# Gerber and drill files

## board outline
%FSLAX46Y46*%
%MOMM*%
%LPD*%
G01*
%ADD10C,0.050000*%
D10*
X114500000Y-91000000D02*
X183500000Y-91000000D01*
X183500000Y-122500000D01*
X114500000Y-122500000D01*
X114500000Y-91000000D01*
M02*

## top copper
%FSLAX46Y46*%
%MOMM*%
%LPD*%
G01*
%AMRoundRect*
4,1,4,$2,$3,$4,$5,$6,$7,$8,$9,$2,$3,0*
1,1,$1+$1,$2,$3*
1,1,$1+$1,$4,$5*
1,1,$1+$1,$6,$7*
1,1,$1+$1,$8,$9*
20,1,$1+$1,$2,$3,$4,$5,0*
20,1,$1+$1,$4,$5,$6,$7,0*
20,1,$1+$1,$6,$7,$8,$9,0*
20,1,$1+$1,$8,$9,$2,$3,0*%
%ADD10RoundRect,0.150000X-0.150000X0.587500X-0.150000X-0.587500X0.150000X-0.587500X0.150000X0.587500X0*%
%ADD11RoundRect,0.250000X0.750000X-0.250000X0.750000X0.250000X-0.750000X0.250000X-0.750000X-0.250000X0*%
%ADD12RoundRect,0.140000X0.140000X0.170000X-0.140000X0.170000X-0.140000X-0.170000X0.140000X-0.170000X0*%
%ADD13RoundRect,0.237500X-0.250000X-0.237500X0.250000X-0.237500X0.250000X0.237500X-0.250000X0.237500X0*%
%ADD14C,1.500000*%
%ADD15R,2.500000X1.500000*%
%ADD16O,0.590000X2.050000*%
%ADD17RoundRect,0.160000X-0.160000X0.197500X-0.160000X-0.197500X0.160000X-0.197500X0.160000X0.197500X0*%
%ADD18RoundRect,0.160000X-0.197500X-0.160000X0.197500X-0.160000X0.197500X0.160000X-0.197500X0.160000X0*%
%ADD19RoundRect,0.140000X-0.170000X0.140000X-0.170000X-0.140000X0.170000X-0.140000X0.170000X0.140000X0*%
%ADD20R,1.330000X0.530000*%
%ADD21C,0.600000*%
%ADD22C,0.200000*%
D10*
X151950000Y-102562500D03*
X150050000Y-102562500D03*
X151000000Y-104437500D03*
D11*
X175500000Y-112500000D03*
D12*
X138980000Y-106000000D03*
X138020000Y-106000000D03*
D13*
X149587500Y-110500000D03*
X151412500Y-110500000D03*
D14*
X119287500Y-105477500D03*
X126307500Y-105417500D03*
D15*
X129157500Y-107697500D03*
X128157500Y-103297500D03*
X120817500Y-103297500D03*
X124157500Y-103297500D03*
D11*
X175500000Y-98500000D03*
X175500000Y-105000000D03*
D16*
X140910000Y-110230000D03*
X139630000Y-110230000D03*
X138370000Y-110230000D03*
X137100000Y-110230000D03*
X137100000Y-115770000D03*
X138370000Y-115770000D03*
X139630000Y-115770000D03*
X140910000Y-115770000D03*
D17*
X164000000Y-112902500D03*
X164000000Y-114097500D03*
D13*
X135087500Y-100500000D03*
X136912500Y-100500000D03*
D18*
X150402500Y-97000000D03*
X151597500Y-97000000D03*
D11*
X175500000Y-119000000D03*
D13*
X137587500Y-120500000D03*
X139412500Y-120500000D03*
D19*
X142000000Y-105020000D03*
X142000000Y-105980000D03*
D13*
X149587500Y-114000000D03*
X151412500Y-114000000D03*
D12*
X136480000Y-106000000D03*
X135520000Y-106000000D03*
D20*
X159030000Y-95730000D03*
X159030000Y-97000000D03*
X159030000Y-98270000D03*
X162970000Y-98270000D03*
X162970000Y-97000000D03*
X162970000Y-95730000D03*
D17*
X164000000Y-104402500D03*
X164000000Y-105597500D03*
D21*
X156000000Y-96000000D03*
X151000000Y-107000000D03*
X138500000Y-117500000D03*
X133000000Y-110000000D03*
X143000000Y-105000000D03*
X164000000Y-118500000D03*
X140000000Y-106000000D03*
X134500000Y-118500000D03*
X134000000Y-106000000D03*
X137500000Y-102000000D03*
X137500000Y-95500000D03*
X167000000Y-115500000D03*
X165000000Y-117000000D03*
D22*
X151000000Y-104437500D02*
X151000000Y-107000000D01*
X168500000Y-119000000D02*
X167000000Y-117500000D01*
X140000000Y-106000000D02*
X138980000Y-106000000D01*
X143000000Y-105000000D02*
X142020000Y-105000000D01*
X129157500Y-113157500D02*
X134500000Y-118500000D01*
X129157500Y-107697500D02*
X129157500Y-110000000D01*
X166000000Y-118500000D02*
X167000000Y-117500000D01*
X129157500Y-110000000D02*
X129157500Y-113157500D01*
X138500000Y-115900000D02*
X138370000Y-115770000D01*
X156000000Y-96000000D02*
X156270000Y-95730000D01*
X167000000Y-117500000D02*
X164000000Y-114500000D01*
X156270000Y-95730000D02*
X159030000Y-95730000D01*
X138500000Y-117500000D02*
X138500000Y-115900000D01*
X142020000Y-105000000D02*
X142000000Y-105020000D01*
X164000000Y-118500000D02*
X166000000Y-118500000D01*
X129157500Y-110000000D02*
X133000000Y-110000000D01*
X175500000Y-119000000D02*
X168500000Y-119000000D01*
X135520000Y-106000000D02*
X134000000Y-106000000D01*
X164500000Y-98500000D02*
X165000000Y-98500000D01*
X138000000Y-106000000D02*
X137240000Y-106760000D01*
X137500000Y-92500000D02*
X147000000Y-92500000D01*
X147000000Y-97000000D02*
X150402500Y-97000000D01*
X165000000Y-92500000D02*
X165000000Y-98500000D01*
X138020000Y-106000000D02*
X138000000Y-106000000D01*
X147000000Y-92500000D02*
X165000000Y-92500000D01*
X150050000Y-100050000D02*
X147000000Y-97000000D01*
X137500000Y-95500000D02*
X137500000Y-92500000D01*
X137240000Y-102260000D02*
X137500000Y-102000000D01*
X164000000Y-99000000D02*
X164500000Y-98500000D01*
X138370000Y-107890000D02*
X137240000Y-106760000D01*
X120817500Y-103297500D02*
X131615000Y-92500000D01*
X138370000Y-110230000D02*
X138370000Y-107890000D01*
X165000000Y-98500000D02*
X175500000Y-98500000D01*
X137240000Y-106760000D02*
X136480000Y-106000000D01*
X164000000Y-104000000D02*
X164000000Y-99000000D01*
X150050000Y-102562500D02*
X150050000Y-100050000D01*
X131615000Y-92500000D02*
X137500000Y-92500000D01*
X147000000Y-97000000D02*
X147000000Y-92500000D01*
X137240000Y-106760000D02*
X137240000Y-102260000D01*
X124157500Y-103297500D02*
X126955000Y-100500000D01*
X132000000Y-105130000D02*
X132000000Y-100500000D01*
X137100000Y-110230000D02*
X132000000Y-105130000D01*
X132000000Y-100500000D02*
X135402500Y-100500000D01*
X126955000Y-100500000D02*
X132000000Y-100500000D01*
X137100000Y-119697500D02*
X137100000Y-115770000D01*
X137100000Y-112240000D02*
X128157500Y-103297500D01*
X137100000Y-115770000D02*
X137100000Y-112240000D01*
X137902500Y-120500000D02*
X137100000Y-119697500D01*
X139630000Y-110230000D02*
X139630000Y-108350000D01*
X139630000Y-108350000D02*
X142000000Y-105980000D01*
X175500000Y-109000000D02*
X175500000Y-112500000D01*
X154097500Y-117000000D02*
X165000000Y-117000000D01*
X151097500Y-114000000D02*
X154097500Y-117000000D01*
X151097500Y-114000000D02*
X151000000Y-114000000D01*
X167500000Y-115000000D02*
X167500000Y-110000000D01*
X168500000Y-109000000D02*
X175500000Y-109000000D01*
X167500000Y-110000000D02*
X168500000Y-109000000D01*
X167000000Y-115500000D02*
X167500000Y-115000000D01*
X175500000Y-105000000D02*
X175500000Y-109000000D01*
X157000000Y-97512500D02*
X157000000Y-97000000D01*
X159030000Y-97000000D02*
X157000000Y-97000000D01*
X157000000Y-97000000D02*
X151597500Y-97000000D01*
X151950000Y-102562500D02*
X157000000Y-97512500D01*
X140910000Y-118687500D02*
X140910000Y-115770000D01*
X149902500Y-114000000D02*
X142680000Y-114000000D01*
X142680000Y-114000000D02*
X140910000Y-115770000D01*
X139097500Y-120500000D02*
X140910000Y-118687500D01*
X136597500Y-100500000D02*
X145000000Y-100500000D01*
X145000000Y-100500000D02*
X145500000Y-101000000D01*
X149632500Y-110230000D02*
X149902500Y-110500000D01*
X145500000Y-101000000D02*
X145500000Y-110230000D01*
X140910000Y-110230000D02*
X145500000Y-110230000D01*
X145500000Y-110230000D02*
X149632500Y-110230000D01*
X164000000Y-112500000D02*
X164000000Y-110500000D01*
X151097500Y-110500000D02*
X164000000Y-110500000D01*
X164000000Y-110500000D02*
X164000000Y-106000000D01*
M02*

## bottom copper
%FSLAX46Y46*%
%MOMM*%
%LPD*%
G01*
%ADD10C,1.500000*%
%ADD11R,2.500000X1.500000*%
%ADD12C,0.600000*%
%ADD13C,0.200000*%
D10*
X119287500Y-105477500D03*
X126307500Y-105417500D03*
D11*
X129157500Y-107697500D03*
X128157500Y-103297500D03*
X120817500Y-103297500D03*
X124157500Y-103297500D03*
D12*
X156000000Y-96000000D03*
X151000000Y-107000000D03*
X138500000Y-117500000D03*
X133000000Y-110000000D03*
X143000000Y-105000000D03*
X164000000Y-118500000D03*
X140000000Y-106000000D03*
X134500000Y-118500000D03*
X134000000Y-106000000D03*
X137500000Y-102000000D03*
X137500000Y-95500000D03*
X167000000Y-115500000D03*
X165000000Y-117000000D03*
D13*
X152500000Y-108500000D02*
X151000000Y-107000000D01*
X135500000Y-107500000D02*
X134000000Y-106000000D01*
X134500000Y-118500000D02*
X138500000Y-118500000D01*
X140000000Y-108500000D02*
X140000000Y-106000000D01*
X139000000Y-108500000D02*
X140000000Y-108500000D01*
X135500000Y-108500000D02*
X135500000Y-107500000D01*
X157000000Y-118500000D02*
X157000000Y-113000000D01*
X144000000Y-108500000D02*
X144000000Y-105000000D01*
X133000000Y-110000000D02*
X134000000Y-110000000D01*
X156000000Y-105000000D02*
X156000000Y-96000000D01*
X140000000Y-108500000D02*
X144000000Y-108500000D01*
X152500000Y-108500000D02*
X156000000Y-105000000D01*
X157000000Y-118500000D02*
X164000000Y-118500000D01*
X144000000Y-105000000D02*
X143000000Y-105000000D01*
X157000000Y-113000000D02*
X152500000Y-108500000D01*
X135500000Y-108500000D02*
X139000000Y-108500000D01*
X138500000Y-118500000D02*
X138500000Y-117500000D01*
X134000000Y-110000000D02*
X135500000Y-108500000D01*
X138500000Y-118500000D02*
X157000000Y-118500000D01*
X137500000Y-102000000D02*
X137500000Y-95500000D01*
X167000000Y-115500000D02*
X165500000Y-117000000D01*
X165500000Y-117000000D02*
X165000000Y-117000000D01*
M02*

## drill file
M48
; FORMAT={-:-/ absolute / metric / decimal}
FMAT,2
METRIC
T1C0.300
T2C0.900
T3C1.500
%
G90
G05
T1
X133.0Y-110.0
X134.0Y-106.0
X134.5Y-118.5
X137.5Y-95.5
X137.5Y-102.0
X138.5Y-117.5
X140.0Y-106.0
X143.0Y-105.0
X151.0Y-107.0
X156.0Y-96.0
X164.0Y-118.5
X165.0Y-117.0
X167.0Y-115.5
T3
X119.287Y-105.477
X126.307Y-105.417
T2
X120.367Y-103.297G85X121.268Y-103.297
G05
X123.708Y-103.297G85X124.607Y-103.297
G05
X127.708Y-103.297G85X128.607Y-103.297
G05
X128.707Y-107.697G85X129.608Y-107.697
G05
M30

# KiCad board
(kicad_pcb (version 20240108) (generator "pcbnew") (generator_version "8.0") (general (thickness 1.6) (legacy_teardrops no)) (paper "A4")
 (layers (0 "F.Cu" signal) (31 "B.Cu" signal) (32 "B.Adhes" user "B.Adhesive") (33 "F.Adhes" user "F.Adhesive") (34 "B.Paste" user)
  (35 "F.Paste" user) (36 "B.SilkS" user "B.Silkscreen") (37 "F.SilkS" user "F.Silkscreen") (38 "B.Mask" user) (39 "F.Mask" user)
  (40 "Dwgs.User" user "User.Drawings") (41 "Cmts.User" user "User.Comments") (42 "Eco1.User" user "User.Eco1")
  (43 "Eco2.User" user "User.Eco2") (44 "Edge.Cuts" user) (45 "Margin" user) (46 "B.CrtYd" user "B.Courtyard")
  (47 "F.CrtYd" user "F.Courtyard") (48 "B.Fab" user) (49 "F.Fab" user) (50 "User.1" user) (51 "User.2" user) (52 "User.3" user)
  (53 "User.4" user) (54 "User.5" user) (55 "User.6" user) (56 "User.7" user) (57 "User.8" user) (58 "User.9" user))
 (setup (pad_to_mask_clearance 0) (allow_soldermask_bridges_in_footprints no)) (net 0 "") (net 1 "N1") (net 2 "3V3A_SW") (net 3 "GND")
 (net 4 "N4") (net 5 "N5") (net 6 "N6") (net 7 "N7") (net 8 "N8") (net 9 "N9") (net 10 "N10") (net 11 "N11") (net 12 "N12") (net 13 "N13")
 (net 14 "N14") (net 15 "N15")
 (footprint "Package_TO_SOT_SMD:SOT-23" (layer "F.Cu") (at 151 103.5 -90)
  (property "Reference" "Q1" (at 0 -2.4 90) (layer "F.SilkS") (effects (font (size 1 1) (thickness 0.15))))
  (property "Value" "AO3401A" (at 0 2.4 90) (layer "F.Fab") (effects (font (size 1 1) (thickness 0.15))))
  (pad "1" smd roundrect (at -0.9375 -0.95 270) (size 1.475 0.6) (layers "F.Cu" "F.Paste" "F.Mask") (roundrect_rratio 0.25) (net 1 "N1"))
  (pad "2" smd roundrect (at -0.9375 0.95 270) (size 1.475 0.6) (layers "F.Cu" "F.Paste" "F.Mask") (roundrect_rratio 0.25) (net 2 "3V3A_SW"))
  (pad "3" smd roundrect (at 0.9375 0 270) (size 1.475 0.6) (layers "F.Cu" "F.Paste" "F.Mask") (roundrect_rratio 0.25) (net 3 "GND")))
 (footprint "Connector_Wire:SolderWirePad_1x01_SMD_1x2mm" (layer "F.Cu") (at 175.5 112.5 90)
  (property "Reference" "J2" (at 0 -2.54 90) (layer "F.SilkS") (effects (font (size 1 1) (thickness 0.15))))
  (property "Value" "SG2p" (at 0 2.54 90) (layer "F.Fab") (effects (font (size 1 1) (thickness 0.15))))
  (pad "1" smd roundrect (at 0 0 90) (size 1 2) (layers "F.Cu" "F.Paste" "F.Mask") (roundrect_rratio 0.25) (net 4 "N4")))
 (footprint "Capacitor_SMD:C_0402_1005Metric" (layer "F.Cu") (at 138.5 106 180)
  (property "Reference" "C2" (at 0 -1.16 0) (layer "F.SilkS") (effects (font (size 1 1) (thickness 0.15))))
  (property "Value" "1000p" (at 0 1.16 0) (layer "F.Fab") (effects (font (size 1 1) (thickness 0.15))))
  (pad "1" smd roundrect (at -0.48 0 180) (size 0.56 0.62) (layers "F.Cu" "F.Paste" "F.Mask") (roundrect_rratio 0.25) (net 3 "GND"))
  (pad "2" smd roundrect (at 0.48 0 180) (size 0.56 0.62) (layers "F.Cu" "F.Paste" "F.Mask") (roundrect_rratio 0.25) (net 2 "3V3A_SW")))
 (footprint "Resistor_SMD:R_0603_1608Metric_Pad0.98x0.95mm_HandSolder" (layer "F.Cu") (at 150.5 110.5)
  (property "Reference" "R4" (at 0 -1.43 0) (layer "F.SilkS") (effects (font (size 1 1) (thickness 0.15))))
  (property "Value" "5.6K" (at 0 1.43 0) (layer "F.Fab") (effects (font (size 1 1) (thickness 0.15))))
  (pad "1" smd roundrect (at -0.9125 0) (size 0.975 0.95) (layers "F.Cu" "F.Paste" "F.Mask") (roundrect_rratio 0.25) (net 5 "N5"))
  (pad "2" smd roundrect (at 0.9125 0) (size 0.975 0.95) (layers "F.Cu" "F.Paste" "F.Mask") (roundrect_rratio 0.25) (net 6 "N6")))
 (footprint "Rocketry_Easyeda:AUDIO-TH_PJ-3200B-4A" (layer "F.Cu") (at 124.9875 105.4975)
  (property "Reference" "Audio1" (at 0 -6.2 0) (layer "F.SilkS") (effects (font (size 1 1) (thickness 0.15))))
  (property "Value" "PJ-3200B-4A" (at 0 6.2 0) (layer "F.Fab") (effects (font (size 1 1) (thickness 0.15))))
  (pad "" thru_hole circle (at -5.7 -0.02) (size 1.5 1.5) (drill 1.5) (layers "*.Cu" "*.Mask") (remove_unused_layers no))
  (pad "" thru_hole circle (at 1.32 -0.08) (size 1.5 1.5) (drill 1.5) (layers "*.Cu" "*.Mask") (remove_unused_layers no))
  (pad "1" thru_hole rect (at 4.17 2.2 90) (size 1.5 2.5) (drill oval 0.900024 1.8002) (layers "*.Cu" "*.Mask") (remove_unused_layers no)
   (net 3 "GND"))
  (pad "2" thru_hole rect (at 3.17 -2.2 90) (size 1.5 2.5) (drill oval 0.900024 1.799946) (layers "*.Cu" "*.Mask") (remove_unused_layers no)
   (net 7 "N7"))
  (pad "3" thru_hole rect (at -4.17 -2.2 90) (size 1.5 2.5) (drill oval 0.900024 1.8002) (layers "*.Cu" "*.Mask") (remove_unused_layers no)
   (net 2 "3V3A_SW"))
  (pad "4" thru_hole rect (at -0.83 -2.2 90) (size 1.5 2.5) (drill oval 0.900024 1.799946) (layers "*.Cu" "*.Mask")
   (remove_unused_layers no) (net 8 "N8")))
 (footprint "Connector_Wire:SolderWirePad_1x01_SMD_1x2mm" (layer "F.Cu") (at 175.5 98.5 90)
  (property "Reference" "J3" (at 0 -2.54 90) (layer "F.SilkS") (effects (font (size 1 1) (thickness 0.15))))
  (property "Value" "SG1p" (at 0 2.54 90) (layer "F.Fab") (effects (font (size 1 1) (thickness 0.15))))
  (pad "1" smd roundrect (at 0 0 90) (size 1 2) (layers "F.Cu" "F.Paste" "F.Mask") (roundrect_rratio 0.25) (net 2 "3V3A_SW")))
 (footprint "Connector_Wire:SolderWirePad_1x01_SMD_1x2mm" (layer "F.Cu") (at 175.5 105 90)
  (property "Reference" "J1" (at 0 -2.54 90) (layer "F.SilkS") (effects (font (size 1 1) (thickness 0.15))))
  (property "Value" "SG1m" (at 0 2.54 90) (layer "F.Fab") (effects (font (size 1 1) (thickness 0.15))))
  (pad "1" smd roundrect (at 0 0 90) (size 1 2) (layers "F.Cu" "F.Paste" "F.Mask") (roundrect_rratio 0.25) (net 4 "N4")))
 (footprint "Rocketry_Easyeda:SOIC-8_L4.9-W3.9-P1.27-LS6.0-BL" (layer "F.Cu") (at 139 113 180)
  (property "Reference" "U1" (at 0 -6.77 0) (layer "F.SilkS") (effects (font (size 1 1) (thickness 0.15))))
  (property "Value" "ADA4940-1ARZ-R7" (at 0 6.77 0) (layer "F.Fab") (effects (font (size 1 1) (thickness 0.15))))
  (pad "1" smd oval (at -1.91 2.77 180) (size 0.59 2.05) (layers "F.Cu" "F.Paste" "F.Mask") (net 5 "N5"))
  (pad "2" smd oval (at -0.63 2.77 180) (size 0.59 2.05) (layers "F.Cu" "F.Paste" "F.Mask") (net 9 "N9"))
  (pad "3" smd oval (at 0.63 2.77 180) (size 0.59 2.05) (layers "F.Cu" "F.Paste" "F.Mask") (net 2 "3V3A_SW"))
  (pad "4" smd oval (at 1.9 2.77 180) (size 0.59 2.05) (layers "F.Cu" "F.Paste" "F.Mask") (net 8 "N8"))
  (pad "5" smd oval (at 1.9 -2.77 180) (size 0.59 2.05) (layers "F.Cu" "F.Paste" "F.Mask") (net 7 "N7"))
  (pad "6" smd oval (at 0.63 -2.77 180) (size 0.59 2.05) (layers "F.Cu" "F.Paste" "F.Mask") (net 3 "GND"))
  (pad "7" smd oval (at -0.63 -2.77 180) (size 0.59 2.05) (layers "F.Cu" "F.Paste" "F.Mask") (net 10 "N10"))
  (pad "8" smd oval (at -1.91 -2.77 180) (size 0.59 2.05) (layers "F.Cu" "F.Paste" "F.Mask") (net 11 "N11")))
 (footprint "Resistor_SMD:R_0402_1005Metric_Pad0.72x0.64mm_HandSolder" (layer "F.Cu") (at 164 113.5 -90)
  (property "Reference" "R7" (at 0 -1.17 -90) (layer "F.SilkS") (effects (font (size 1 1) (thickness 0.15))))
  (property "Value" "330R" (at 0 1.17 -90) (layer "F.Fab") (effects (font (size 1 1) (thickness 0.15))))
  (pad "1" smd roundrect (at -0.5975 0 270) (size 0.715 0.64) (layers "F.Cu" "F.Paste" "F.Mask") (roundrect_rratio 0.25) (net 6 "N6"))
  (pad "2" smd roundrect (at 0.5975 0 270) (size 0.715 0.64) (layers "F.Cu" "F.Paste" "F.Mask") (roundrect_rratio 0.25) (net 3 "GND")))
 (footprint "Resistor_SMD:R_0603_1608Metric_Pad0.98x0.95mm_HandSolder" (layer "F.Cu") (at 136 100.5)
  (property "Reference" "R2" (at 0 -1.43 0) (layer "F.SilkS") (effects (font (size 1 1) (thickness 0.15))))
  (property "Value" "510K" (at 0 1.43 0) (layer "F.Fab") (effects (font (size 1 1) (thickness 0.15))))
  (pad "1" smd roundrect (at -0.9125 0) (size 0.975 0.95) (layers "F.Cu" "F.Paste" "F.Mask") (roundrect_rratio 0.25) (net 8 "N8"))
  (pad "2" smd roundrect (at 0.9125 0) (size 0.975 0.95) (layers "F.Cu" "F.Paste" "F.Mask") (roundrect_rratio 0.25) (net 5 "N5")))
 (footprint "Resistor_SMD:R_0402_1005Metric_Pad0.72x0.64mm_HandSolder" (layer "F.Cu") (at 151 97)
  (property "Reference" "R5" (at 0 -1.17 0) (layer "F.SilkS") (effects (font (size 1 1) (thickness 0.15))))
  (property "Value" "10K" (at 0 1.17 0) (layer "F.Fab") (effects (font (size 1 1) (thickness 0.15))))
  (pad "1" smd roundrect (at -0.5975 0) (size 0.715 0.64) (layers "F.Cu" "F.Paste" "F.Mask") (roundrect_rratio 0.25) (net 2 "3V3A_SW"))
  (pad "2" smd roundrect (at 0.5975 0) (size 0.715 0.64) (layers "F.Cu" "F.Paste" "F.Mask") (roundrect_rratio 0.25) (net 1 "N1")))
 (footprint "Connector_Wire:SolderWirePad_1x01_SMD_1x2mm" (layer "F.Cu") (at 175.5 119 90)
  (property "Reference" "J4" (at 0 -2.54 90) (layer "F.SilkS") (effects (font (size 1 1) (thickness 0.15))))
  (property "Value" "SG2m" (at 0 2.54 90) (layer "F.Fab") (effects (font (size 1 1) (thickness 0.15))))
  (pad "1" smd roundrect (at 0 0 90) (size 1 2) (layers "F.Cu" "F.Paste" "F.Mask") (roundrect_rratio 0.25) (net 3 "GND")))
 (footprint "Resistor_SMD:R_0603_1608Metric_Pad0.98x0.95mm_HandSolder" (layer "F.Cu") (at 138.5 120.5)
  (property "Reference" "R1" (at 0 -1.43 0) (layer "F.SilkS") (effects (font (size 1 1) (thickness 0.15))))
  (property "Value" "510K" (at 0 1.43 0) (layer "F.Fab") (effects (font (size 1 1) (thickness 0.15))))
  (pad "1" smd roundrect (at -0.9125 0) (size 0.975 0.95) (layers "F.Cu" "F.Paste" "F.Mask") (roundrect_rratio 0.25) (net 7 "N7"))
  (pad "2" smd roundrect (at 0.9125 0) (size 0.975 0.95) (layers "F.Cu" "F.Paste" "F.Mask") (roundrect_rratio 0.25) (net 11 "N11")))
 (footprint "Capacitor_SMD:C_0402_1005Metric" (layer "F.Cu") (at 142 105.5 -90)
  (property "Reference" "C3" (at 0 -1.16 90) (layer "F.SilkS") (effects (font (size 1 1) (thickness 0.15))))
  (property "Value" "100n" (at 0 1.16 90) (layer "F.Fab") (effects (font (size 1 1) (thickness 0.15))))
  (pad "1" smd roundrect (at -0.48 0 270) (size 0.56 0.62) (layers "F.Cu" "F.Paste" "F.Mask") (roundrect_rratio 0.25) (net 3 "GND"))
  (pad "2" smd roundrect (at 0.48 0 270) (size 0.56 0.62) (layers "F.Cu" "F.Paste" "F.Mask") (roundrect_rratio 0.25) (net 9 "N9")))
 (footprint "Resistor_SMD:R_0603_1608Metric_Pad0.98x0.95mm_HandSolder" (layer "F.Cu") (at 150.5 114)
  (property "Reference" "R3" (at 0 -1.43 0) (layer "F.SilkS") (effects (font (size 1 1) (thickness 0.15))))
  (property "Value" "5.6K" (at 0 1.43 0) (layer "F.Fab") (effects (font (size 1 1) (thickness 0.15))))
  (pad "1" smd roundrect (at -0.9125 0) (size 0.975 0.95) (layers "F.Cu" "F.Paste" "F.Mask") (roundrect_rratio 0.25) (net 11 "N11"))
  (pad "2" smd roundrect (at 0.9125 0) (size 0.975 0.95) (layers "F.Cu" "F.Paste" "F.Mask") (roundrect_rratio 0.25) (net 4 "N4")))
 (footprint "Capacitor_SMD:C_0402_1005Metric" (layer "F.Cu") (at 136 106 180)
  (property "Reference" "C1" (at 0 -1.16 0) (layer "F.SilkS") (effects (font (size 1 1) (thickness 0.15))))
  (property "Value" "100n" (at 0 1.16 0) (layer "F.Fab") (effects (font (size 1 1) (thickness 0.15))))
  (pad "1" smd roundrect (at -0.48 0 180) (size 0.56 0.62) (layers "F.Cu" "F.Paste" "F.Mask") (roundrect_rratio 0.25) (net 2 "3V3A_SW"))
  (pad "2" smd roundrect (at 0.48 0 180) (size 0.56 0.62) (layers "F.Cu" "F.Paste" "F.Mask") (roundrect_rratio 0.25) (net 3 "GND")))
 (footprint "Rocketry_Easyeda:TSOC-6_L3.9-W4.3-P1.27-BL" (layer "F.Cu") (at 161 97 -90)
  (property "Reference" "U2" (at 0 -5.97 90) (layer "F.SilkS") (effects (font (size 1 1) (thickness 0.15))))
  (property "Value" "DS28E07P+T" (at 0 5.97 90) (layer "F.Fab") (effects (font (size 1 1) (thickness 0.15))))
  (pad "1" smd rect (at -1.27 1.97 270) (size 0.53 1.33) (layers "F.Cu" "F.Paste" "F.Mask") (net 3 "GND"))
  (pad "2" smd rect (at 0 1.97 270) (size 0.53 1.33) (layers "F.Cu" "F.Paste" "F.Mask") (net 1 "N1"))
  (pad "3" smd rect (at 1.27 1.97 270) (size 0.53 1.33) (layers "F.Cu" "F.Paste" "F.Mask") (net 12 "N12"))
  (pad "4" smd rect (at 1.27 -1.97 270) (size 0.53 1.33) (layers "F.Cu" "F.Paste" "F.Mask") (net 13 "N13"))
  (pad "5" smd rect (at 0 -1.97 270) (size 0.53 1.33) (layers "F.Cu" "F.Paste" "F.Mask") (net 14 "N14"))
  (pad "6" smd rect (at -1.27 -1.97 270) (size 0.53 1.33) (layers "F.Cu" "F.Paste" "F.Mask") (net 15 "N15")))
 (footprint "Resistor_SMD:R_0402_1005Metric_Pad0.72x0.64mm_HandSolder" (layer "F.Cu") (at 164 105 -90)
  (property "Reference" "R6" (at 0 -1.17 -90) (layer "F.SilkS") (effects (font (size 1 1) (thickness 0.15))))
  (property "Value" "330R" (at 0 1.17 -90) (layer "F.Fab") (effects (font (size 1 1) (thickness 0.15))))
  (pad "1" smd roundrect (at -0.5975 0 270) (size 0.715 0.64) (layers "F.Cu" "F.Paste" "F.Mask") (roundrect_rratio 0.25) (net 2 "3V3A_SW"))
  (pad "2" smd roundrect (at 0.5975 0 270) (size 0.715 0.64) (layers "F.Cu" "F.Paste" "F.Mask") (roundrect_rratio 0.25) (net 6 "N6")))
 (gr_rect (start 114.5 91) (end 183.5 122.5) (stroke (width 0.05) (type default)) (fill none) (layer "Edge.Cuts"))
 (segment (start 151 104.4375) (end 151 107) (width 0.2) (layer "F.Cu") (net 3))
 (segment (start 168.5 119) (end 167 117.5) (width 0.2) (layer "F.Cu") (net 3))
 (segment (start 140 106) (end 138.98 106) (width 0.2) (layer "F.Cu") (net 3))
 (segment (start 143 105) (end 142.02 105) (width 0.2) (layer "F.Cu") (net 3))
 (segment (start 129.1575 113.1575) (end 134.5 118.5) (width 0.2) (layer "F.Cu") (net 3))
 (segment (start 129.1575 107.6975) (end 129.1575 110) (width 0.2) (layer "F.Cu") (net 3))
 (segment (start 166 118.5) (end 167 117.5) (width 0.2) (layer "F.Cu") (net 3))
 (segment (start 129.1575 110) (end 129.1575 113.1575) (width 0.2) (layer "F.Cu") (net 3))
 (segment (start 138.5 115.9) (end 138.37 115.77) (width 0.2) (layer "F.Cu") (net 3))
 (segment (start 156 96) (end 156.27 95.73) (width 0.2) (layer "F.Cu") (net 3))
 (segment (start 167 117.5) (end 164 114.5) (width 0.2) (layer "F.Cu") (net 3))
 (segment (start 156.27 95.73) (end 159.03 95.73) (width 0.2) (layer "F.Cu") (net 3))
 (segment (start 138.5 117.5) (end 138.5 115.9) (width 0.2) (layer "F.Cu") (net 3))
 (segment (start 142.02 105) (end 142 105.02) (width 0.2) (layer "F.Cu") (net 3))
 (segment (start 164 118.5) (end 166 118.5) (width 0.2) (layer "F.Cu") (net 3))
 (segment (start 129.1575 110) (end 133 110) (width 0.2) (layer "F.Cu") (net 3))
 (segment (start 175.5 119) (end 168.5 119) (width 0.2) (layer "F.Cu") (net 3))
 (segment (start 135.52 106) (end 134 106) (width 0.2) (layer "F.Cu") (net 3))
 (via (at 156 96) (size 0.6) (drill 0.3) (layers "F.Cu" "B.Cu") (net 3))
 (via (at 151 107) (size 0.6) (drill 0.3) (layers "F.Cu" "B.Cu") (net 3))
 (via (at 138.5 117.5) (size 0.6) (drill 0.3) (layers "F.Cu" "B.Cu") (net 3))
 (via (at 133 110) (size 0.6) (drill 0.3) (layers "F.Cu" "B.Cu") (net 3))
 (via (at 143 105) (size 0.6) (drill 0.3) (layers "F.Cu" "B.Cu") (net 3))
 (via (at 164 118.5) (size 0.6) (drill 0.3) (layers "F.Cu" "B.Cu") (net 3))
 (via (at 140 106) (size 0.6) (drill 0.3) (layers "F.Cu" "B.Cu") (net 3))
 (via (at 134.5 118.5) (size 0.6) (drill 0.3) (layers "F.Cu" "B.Cu") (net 3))
 (via (at 134 106) (size 0.6) (drill 0.3) (layers "F.Cu" "B.Cu") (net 3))
 (segment (start 152.5 108.5) (end 151 107) (width 0.2) (layer "B.Cu") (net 3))
 (segment (start 135.5 107.5) (end 134 106) (width 0.2) (layer "B.Cu") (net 3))
 (segment (start 134.5 118.5) (end 138.5 118.5) (width 0.2) (layer "B.Cu") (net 3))
 (segment (start 140 108.5) (end 140 106) (width 0.2) (layer "B.Cu") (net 3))
 (segment (start 139 108.5) (end 140 108.5) (width 0.2) (layer "B.Cu") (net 3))
 (segment (start 135.5 108.5) (end 135.5 107.5) (width 0.2) (layer "B.Cu") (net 3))
 (segment (start 157 118.5) (end 157 113) (width 0.2) (layer "B.Cu") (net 3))
 (segment (start 144 108.5) (end 144 105) (width 0.2) (layer "B.Cu") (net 3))
 (segment (start 133 110) (end 134 110) (width 0.2) (layer "B.Cu") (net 3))
 (segment (start 156 105) (end 156 96) (width 0.2) (layer "B.Cu") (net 3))
 (segment (start 140 108.5) (end 144 108.5) (width 0.2) (layer "B.Cu") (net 3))
 (segment (start 152.5 108.5) (end 156 105) (width 0.2) (layer "B.Cu") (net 3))
 (segment (start 157 118.5) (end 164 118.5) (width 0.2) (layer "B.Cu") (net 3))
 (segment (start 144 105) (end 143 105) (width 0.2) (layer "B.Cu") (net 3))
 (segment (start 157 113) (end 152.5 108.5) (width 0.2) (layer "B.Cu") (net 3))
 (segment (start 135.5 108.5) (end 139 108.5) (width 0.2) (layer "B.Cu") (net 3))
 (segment (start 138.5 118.5) (end 138.5 117.5) (width 0.2) (layer "B.Cu") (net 3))
 (segment (start 134 110) (end 135.5 108.5) (width 0.2) (layer "B.Cu") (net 3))
 (segment (start 138.5 118.5) (end 157 118.5) (width 0.2) (layer "B.Cu") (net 3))
 (segment (start 164.5 98.5) (end 165 98.5) (width 0.2) (layer "F.Cu") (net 2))
 (segment (start 138 106) (end 137.24 106.76) (width 0.2) (layer "F.Cu") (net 2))
 (segment (start 137.5 92.5) (end 147 92.5) (width 0.2) (layer "F.Cu") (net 2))
 (segment (start 147 97) (end 150.4025 97) (width 0.2) (layer "F.Cu") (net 2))
 (segment (start 165 92.5) (end 165 98.5) (width 0.2) (layer "F.Cu") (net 2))
 (segment (start 138.02 106) (end 138 106) (width 0.2) (layer "F.Cu") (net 2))
 (segment (start 147 92.5) (end 165 92.5) (width 0.2) (layer "F.Cu") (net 2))
 (segment (start 150.05 100.05) (end 147 97) (width 0.2) (layer "F.Cu") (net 2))
 (segment (start 137.5 95.5) (end 137.5 92.5) (width 0.2) (layer "F.Cu") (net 2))
 (segment (start 137.24 102.26) (end 137.5 102) (width 0.2) (layer "F.Cu") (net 2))
 (segment (start 164 99) (end 164.5 98.5) (width 0.2) (layer "F.Cu") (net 2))
 (segment (start 138.37 107.89) (end 137.24 106.76) (width 0.2) (layer "F.Cu") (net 2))
 (segment (start 120.8175 103.2975) (end 131.615 92.5) (width 0.2) (layer "F.Cu") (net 2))
 (segment (start 138.37 110.23) (end 138.37 107.89) (width 0.2) (layer "F.Cu") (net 2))
 (segment (start 165 98.5) (end 175.5 98.5) (width 0.2) (layer "F.Cu") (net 2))
 (segment (start 137.24 106.76) (end 136.48 106) (width 0.2) (layer "F.Cu") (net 2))
 (segment (start 164 104) (end 164 99) (width 0.2) (layer "F.Cu") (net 2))
 (segment (start 150.05 102.5625) (end 150.05 100.05) (width 0.2) (layer "F.Cu") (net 2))
 (segment (start 131.615 92.5) (end 137.5 92.5) (width 0.2) (layer "F.Cu") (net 2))
 (segment (start 147 97) (end 147 92.5) (width 0.2) (layer "F.Cu") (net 2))
 (segment (start 137.24 106.76) (end 137.24 102.26) (width 0.2) (layer "F.Cu") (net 2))
 (via (at 137.5 102) (size 0.6) (drill 0.3) (layers "F.Cu" "B.Cu") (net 2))
 (via (at 137.5 95.5) (size 0.6) (drill 0.3) (layers "F.Cu" "B.Cu") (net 2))
 (segment (start 137.5 102) (end 137.5 95.5) (width 0.2) (layer "B.Cu") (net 2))
 (segment (start 124.1575 103.2975) (end 126.955 100.5) (width 0.2) (layer "F.Cu") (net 8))
 (segment (start 132 105.13) (end 132 100.5) (width 0.2) (layer "F.Cu") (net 8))
 (segment (start 137.1 110.23) (end 132 105.13) (width 0.2) (layer "F.Cu") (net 8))
 (segment (start 132 100.5) (end 135.4025 100.5) (width 0.2) (layer "F.Cu") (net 8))
 (segment (start 126.955 100.5) (end 132 100.5) (width 0.2) (layer "F.Cu") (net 8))
 (segment (start 137.1 119.6975) (end 137.1 115.77) (width 0.2) (layer "F.Cu") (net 7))
 (segment (start 137.1 112.24) (end 128.1575 103.2975) (width 0.2) (layer "F.Cu") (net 7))
 (segment (start 137.1 115.77) (end 137.1 112.24) (width 0.2) (layer "F.Cu") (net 7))
 (segment (start 137.9025 120.5) (end 137.1 119.6975) (width 0.2) (layer "F.Cu") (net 7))
 (segment (start 139.63 110.23) (end 139.63 108.35) (width 0.2) (layer "F.Cu") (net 9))
 (segment (start 139.63 108.35) (end 142 105.98) (width 0.2) (layer "F.Cu") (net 9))
 (segment (start 175.5 109) (end 175.5 112.5) (width 0.2) (layer "F.Cu") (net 4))
 (segment (start 154.0975 117) (end 165 117) (width 0.2) (layer "F.Cu") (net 4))
 (segment (start 151.0975 114) (end 154.0975 117) (width 0.2) (layer "F.Cu") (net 4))
 (segment (start 151.0975 114) (end 151 114) (width 0.2) (layer "F.Cu") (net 4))
 (segment (start 167.5 115) (end 167.5 110) (width 0.2) (layer "F.Cu") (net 4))
 (segment (start 168.5 109) (end 175.5 109) (width 0.2) (layer "F.Cu") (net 4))
 (segment (start 167.5 110) (end 168.5 109) (width 0.2) (layer "F.Cu") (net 4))
 (segment (start 167 115.5) (end 167.5 115) (width 0.2) (layer "F.Cu") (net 4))
 (segment (start 175.5 105) (end 175.5 109) (width 0.2) (layer "F.Cu") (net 4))
 (via (at 167 115.5) (size 0.6) (drill 0.3) (layers "F.Cu" "B.Cu") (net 4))
 (via (at 165 117) (size 0.6) (drill 0.3) (layers "F.Cu" "B.Cu") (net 4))
 (segment (start 167 115.5) (end 165.5 117) (width 0.2) (layer "B.Cu") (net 4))
 (segment (start 165.5 117) (end 165 117) (width 0.2) (layer "B.Cu") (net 4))
 (segment (start 157 97.5125) (end 157 97) (width 0.2) (layer "F.Cu") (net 1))
 (segment (start 159.03 97) (end 157 97) (width 0.2) (layer "F.Cu") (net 1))
 (segment (start 157 97) (end 151.5975 97) (width 0.2) (layer "F.Cu") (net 1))
 (segment (start 151.95 102.5625) (end 157 97.5125) (width 0.2) (layer "F.Cu") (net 1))
 (segment (start 140.91 118.6875) (end 140.91 115.77) (width 0.2) (layer "F.Cu") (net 11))
 (segment (start 149.9025 114) (end 142.68 114) (width 0.2) (layer "F.Cu") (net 11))
 (segment (start 142.68 114) (end 140.91 115.77) (width 0.2) (layer "F.Cu") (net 11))
 (segment (start 139.0975 120.5) (end 140.91 118.6875) (width 0.2) (layer "F.Cu") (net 11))
 (segment (start 136.5975 100.5) (end 145 100.5) (width 0.2) (layer "F.Cu") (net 5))
 (segment (start 145 100.5) (end 145.5 101) (width 0.2) (layer "F.Cu") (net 5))
 (segment (start 149.6325 110.23) (end 149.9025 110.5) (width 0.2) (layer "F.Cu") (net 5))
 (segment (start 145.5 101) (end 145.5 110.23) (width 0.2) (layer "F.Cu") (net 5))
 (segment (start 140.91 110.23) (end 145.5 110.23) (width 0.2) (layer "F.Cu") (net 5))
 (segment (start 145.5 110.23) (end 149.6325 110.23) (width 0.2) (layer "F.Cu") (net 5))
 (segment (start 164 112.5) (end 164 110.5) (width 0.2) (layer "F.Cu") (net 6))
 (segment (start 151.0975 110.5) (end 164 110.5) (width 0.2) (layer "F.Cu") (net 6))
 (segment (start 164 110.5) (end 164 106) (width 0.2) (layer "F.Cu") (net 6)))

